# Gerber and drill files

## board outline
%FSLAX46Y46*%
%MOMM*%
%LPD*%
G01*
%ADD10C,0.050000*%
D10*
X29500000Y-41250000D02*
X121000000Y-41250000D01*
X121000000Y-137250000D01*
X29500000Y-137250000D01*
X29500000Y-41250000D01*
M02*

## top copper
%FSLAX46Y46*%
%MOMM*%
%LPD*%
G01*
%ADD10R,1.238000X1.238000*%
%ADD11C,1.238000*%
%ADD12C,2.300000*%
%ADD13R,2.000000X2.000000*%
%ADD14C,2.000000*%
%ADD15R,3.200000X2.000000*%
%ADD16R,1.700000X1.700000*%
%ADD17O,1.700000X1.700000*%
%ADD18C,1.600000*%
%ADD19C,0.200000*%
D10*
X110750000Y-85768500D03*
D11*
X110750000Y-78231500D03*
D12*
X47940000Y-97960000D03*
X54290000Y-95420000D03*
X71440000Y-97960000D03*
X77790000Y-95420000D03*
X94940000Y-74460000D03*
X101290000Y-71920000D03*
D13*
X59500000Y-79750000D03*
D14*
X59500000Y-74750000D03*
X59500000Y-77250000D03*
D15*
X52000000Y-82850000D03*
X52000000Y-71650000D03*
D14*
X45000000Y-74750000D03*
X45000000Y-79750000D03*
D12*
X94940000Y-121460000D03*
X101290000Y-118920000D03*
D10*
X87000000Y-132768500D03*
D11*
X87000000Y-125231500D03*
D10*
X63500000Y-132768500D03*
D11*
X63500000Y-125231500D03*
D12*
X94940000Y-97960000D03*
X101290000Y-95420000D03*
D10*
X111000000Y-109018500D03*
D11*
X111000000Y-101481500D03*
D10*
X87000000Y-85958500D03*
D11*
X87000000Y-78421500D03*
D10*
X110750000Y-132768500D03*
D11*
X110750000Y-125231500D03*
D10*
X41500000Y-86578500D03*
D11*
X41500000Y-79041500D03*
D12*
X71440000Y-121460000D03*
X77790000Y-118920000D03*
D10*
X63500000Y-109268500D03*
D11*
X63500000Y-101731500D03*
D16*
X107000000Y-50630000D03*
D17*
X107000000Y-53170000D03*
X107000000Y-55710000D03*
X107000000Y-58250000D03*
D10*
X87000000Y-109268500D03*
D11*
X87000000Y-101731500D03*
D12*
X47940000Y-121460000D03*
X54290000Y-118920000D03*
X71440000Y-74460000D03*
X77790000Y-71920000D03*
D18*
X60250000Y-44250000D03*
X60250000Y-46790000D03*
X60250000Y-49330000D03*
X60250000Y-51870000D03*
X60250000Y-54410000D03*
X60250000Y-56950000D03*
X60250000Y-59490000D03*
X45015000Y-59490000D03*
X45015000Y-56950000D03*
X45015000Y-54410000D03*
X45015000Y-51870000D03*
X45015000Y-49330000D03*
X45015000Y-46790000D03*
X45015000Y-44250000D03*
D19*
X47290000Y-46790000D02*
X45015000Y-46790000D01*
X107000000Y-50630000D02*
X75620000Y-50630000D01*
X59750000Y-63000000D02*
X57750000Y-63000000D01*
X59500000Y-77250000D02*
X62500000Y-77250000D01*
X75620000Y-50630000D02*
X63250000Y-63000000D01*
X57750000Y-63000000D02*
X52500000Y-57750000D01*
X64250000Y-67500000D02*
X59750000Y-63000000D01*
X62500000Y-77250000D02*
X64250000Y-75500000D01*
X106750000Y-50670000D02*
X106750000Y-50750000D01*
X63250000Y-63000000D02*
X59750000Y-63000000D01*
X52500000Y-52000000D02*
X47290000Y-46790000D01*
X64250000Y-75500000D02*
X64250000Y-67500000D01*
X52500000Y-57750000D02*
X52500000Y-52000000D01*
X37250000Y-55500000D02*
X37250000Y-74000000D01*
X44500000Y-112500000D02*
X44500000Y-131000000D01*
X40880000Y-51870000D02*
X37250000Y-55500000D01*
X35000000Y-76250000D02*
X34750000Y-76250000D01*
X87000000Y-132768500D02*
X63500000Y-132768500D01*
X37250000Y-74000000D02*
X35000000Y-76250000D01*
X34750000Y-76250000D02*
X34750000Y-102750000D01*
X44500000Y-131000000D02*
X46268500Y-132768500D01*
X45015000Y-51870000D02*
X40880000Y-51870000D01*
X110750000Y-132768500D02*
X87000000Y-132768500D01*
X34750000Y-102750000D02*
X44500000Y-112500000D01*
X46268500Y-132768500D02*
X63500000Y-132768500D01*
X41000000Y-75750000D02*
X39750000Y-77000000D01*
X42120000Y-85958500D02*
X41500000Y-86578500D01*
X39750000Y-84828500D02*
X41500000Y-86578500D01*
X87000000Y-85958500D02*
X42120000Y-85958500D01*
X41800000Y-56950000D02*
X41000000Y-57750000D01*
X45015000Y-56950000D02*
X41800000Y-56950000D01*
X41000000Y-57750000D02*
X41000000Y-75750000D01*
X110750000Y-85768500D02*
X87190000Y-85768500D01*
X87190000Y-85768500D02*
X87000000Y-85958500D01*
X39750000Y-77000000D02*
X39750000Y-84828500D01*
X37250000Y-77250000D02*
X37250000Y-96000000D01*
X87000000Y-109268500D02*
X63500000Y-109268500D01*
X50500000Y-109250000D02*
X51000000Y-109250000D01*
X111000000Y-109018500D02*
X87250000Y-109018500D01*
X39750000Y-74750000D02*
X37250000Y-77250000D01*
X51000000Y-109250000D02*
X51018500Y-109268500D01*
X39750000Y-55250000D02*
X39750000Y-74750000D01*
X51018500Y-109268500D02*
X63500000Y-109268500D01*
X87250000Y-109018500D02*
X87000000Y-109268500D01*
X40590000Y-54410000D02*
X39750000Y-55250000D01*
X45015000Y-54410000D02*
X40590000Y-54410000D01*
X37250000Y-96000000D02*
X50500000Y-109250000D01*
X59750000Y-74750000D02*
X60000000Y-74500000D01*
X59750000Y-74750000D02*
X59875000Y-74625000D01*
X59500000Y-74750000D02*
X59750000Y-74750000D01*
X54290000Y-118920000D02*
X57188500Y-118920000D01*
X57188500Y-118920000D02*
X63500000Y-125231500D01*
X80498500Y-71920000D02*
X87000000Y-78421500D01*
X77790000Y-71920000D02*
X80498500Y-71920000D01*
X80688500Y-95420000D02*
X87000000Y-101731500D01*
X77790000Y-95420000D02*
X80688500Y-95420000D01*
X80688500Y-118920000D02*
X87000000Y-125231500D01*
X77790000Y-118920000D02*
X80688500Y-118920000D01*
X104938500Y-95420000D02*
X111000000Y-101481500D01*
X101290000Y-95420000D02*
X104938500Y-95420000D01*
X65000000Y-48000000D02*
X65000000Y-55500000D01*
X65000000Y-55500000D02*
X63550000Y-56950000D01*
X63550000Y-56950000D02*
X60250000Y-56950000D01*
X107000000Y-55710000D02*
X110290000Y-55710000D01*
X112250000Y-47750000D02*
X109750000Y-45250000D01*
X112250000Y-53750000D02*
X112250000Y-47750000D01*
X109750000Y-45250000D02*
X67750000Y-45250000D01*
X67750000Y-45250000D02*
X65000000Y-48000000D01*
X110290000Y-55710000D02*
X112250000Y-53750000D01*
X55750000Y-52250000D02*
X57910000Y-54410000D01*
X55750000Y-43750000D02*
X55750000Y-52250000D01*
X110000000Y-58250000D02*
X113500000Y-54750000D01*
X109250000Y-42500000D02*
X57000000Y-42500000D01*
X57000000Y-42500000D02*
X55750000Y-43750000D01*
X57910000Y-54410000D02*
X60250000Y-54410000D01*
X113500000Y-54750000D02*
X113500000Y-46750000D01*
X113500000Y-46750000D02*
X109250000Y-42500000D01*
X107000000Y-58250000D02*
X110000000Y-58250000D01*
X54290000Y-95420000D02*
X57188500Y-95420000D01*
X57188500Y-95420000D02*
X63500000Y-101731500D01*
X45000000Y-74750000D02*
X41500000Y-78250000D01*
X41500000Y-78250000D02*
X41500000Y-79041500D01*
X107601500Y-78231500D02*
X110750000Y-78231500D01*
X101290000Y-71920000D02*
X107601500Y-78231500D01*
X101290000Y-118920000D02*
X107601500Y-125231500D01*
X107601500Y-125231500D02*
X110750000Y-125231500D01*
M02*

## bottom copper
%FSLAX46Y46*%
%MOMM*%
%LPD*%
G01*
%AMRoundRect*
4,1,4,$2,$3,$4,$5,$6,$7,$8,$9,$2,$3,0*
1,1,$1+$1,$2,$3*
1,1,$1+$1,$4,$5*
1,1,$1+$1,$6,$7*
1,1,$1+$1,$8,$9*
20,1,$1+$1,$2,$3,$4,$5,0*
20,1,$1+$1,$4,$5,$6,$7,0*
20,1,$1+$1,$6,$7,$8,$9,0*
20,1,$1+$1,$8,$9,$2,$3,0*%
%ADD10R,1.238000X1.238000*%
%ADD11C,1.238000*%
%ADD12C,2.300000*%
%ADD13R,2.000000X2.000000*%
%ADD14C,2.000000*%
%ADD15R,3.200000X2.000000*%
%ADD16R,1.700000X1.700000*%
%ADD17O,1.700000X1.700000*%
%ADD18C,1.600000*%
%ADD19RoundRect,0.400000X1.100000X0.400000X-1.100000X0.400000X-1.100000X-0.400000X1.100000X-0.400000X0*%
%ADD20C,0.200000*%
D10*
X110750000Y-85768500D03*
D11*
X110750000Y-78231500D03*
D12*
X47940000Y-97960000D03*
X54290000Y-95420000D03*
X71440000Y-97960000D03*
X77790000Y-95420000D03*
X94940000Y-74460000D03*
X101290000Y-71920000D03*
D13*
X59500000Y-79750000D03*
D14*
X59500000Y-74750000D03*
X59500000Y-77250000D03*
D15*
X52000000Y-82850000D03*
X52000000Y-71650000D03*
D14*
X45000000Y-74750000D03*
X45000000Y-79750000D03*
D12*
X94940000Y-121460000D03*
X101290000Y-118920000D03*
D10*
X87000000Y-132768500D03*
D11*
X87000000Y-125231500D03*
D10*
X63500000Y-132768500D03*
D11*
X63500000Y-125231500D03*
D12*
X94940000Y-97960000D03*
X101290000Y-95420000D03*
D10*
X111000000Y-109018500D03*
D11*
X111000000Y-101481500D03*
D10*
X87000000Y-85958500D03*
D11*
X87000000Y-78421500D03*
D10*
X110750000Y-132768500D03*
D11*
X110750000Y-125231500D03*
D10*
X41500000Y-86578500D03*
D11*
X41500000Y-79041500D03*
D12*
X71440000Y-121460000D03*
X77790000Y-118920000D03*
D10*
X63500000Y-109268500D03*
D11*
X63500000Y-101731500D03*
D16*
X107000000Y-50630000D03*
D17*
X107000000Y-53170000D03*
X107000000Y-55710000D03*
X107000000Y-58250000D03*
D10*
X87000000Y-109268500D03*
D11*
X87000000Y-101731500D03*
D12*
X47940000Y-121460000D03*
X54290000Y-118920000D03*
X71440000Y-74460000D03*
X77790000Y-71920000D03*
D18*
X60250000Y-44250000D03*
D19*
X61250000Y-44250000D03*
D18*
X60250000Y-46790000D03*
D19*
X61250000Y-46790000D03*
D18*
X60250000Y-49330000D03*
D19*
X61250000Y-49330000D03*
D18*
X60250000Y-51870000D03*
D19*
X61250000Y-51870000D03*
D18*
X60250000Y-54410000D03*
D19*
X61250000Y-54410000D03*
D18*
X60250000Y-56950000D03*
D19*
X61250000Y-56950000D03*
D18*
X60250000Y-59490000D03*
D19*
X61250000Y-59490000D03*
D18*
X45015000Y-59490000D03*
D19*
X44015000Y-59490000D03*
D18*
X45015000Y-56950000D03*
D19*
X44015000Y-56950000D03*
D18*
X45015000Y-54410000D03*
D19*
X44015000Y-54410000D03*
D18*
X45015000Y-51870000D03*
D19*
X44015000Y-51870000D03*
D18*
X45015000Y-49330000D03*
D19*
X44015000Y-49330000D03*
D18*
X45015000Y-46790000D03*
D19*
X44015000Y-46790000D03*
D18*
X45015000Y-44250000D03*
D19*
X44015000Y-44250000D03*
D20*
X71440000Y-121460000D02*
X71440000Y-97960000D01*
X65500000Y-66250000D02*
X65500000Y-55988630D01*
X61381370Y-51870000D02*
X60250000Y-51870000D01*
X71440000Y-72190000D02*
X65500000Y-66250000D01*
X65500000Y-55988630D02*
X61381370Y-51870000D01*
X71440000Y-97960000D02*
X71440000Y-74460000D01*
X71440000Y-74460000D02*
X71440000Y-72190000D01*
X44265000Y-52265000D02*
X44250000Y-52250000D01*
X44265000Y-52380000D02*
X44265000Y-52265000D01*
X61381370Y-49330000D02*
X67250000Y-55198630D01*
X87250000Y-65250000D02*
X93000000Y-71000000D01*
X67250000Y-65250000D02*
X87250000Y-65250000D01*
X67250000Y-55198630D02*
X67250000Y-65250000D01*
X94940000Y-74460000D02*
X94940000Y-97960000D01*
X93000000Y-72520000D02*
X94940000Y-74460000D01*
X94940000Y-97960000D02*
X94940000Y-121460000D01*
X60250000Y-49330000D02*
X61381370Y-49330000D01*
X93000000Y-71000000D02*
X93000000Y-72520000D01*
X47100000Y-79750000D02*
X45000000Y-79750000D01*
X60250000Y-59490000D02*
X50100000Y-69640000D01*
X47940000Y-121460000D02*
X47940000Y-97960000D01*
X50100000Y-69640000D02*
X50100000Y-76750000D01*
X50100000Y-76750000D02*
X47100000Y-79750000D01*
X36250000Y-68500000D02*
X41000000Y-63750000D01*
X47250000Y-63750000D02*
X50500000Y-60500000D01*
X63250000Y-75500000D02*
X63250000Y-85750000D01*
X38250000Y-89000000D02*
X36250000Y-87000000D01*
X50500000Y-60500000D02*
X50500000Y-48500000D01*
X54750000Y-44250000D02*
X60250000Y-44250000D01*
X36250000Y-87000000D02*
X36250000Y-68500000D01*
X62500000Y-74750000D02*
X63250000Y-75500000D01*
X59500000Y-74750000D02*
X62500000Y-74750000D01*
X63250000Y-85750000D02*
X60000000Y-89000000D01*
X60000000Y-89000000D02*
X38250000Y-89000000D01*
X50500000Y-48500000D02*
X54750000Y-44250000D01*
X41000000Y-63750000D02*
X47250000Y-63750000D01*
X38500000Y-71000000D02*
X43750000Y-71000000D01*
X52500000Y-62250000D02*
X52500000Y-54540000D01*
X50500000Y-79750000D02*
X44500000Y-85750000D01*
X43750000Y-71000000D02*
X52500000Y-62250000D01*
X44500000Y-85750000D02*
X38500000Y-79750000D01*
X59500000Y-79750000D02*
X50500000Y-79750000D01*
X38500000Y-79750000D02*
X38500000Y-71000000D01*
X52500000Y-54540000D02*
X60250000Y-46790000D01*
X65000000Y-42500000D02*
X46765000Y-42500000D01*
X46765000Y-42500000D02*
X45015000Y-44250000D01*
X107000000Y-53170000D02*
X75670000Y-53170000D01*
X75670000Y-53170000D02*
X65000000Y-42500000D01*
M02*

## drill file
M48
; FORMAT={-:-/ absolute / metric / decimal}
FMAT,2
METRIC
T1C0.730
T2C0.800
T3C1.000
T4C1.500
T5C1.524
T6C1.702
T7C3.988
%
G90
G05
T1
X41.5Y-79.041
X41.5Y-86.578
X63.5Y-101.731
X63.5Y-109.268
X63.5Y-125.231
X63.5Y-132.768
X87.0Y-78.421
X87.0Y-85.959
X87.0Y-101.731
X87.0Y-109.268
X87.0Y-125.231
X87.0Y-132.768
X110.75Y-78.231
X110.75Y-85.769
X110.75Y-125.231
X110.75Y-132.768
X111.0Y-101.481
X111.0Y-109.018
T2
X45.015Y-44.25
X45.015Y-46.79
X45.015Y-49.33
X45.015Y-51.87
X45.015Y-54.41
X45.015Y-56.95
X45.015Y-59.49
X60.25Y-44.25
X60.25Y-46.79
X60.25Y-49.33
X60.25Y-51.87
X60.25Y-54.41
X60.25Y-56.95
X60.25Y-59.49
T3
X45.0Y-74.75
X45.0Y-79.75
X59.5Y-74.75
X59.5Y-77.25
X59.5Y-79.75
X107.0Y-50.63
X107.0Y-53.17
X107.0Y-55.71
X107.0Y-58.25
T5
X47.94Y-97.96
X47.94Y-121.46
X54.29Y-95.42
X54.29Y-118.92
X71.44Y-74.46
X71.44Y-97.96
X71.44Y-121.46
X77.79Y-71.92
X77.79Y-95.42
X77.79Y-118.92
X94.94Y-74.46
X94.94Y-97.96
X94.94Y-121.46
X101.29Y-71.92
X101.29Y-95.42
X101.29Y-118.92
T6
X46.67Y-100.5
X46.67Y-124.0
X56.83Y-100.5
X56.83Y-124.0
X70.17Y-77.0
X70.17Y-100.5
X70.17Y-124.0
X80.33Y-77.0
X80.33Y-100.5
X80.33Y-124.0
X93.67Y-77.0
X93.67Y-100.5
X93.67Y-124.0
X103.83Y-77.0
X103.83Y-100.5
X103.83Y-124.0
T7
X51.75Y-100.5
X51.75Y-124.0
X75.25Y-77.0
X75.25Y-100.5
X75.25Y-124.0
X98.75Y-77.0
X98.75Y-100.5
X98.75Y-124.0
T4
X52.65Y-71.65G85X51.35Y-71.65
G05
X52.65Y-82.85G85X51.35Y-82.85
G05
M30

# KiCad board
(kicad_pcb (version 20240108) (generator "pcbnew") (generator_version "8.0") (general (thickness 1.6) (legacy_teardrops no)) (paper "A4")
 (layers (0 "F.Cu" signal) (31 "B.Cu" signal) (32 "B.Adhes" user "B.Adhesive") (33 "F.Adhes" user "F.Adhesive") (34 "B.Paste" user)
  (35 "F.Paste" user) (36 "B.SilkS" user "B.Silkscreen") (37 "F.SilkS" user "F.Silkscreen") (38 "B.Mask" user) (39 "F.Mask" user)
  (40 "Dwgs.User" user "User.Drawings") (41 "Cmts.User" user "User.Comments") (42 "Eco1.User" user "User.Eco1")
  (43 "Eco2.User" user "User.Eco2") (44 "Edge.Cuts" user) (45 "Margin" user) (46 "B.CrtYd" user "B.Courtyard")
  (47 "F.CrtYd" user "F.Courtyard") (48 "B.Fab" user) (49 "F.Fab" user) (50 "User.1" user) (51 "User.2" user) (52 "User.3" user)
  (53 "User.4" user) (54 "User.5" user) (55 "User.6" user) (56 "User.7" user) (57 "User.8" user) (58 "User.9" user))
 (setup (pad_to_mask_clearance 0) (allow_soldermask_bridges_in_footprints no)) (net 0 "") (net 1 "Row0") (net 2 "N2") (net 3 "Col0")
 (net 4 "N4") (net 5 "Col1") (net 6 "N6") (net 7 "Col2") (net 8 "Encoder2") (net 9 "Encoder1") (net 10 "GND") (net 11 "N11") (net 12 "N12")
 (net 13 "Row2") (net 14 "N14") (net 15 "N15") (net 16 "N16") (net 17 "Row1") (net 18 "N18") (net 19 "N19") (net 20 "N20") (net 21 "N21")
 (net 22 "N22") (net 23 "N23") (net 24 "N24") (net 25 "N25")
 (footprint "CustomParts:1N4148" (layer "F.Cu") (at 110.75 82 90)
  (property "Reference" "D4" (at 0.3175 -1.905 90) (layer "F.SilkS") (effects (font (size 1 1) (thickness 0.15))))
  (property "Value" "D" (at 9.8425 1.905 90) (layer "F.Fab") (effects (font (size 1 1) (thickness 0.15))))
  (pad "1" thru_hole rect (at -3.7685 0 90) (size 1.238 1.238) (drill 0.73) (layers "*.Cu" "*.Mask") (remove_unused_layers no)
   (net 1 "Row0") (solder_mask_margin 0.102))
  (pad "2" thru_hole circle (at 3.7685 0 90) (size 1.238 1.238) (drill 0.73) (layers "*.Cu" "*.Mask") (remove_unused_layers no) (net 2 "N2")
   (solder_mask_margin 0.102)))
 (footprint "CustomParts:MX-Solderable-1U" (layer "F.Cu") (at 51.75 100.5)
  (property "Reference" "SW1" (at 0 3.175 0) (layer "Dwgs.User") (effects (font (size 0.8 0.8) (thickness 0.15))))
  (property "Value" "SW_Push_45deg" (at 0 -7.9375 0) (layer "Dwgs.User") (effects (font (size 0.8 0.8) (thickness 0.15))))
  (pad "" np_thru_hole circle (at -5.08 0 48.099) (size 1.7018 1.7018) (drill 1.7018) (layers "F&B.Cu" "*.Mask"))
  (pad "" np_thru_hole circle (at 0 0) (size 3.9878 3.9878) (drill 3.9878) (layers "*.Cu" "*.Mask"))
  (pad "" np_thru_hole circle (at 5.08 0 48.099) (size 1.7018 1.7018) (drill 1.7018) (layers "F&B.Cu" "*.Mask"))
  (pad "1" thru_hole circle (at -3.81 -2.54) (size 2.3 2.3) (drill 1.524) (layers "*.Cu" "B.Mask") (remove_unused_layers no) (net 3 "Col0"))
  (pad "2" thru_hole circle (at 2.54 -5.08) (size 2.3 2.3) (drill 1.524) (layers "*.Cu" "B.Mask") (remove_unused_layers no) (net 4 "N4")))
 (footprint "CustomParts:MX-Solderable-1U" (layer "F.Cu") (at 75.25 100.5)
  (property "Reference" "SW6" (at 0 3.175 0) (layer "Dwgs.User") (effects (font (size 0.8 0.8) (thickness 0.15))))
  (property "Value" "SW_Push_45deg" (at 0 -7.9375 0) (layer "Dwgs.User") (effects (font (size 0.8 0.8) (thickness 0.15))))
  (pad "" np_thru_hole circle (at -5.08 0 48.099) (size 1.7018 1.7018) (drill 1.7018) (layers "F&B.Cu" "*.Mask"))
  (pad "" np_thru_hole circle (at 0 0) (size 3.9878 3.9878) (drill 3.9878) (layers "*.Cu" "*.Mask"))
  (pad "" np_thru_hole circle (at 5.08 0 48.099) (size 1.7018 1.7018) (drill 1.7018) (layers "F&B.Cu" "*.Mask"))
  (pad "1" thru_hole circle (at -3.81 -2.54) (size 2.3 2.3) (drill 1.524) (layers "*.Cu" "B.Mask") (remove_unused_layers no) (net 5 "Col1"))
  (pad "2" thru_hole circle (at 2.54 -5.08) (size 2.3 2.3) (drill 1.524) (layers "*.Cu" "B.Mask") (remove_unused_layers no) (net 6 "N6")))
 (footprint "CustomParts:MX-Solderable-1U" (layer "F.Cu") (at 98.75 77)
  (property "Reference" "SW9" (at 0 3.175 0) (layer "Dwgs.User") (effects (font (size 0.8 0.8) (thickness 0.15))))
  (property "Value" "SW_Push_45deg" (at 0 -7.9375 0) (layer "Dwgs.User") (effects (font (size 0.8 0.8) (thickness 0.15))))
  (pad "" np_thru_hole circle (at -5.08 0 48.099) (size 1.7018 1.7018) (drill 1.7018) (layers "F&B.Cu" "*.Mask"))
  (pad "" np_thru_hole circle (at 0 0) (size 3.9878 3.9878) (drill 3.9878) (layers "*.Cu" "*.Mask"))
  (pad "" np_thru_hole circle (at 5.08 0 48.099) (size 1.7018 1.7018) (drill 1.7018) (layers "F&B.Cu" "*.Mask"))
  (pad "1" thru_hole circle (at -3.81 -2.54) (size 2.3 2.3) (drill 1.524) (layers "*.Cu" "B.Mask") (remove_unused_layers no) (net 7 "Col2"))
  (pad "2" thru_hole circle (at 2.54 -5.08) (size 2.3 2.3) (drill 1.524) (layers "*.Cu" "B.Mask") (remove_unused_layers no) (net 2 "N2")))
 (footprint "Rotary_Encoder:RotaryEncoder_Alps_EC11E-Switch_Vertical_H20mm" (layer "F.Cu") (at 59.5 79.75 180)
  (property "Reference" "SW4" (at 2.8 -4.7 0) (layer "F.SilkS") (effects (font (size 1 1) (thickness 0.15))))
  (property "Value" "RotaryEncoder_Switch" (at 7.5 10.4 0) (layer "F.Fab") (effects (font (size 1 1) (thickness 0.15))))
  (pad "A" thru_hole rect (at 0 0 180) (size 2 2) (drill 1) (layers "*.Cu" "*.Mask") (remove_unused_layers no) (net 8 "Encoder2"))
  (pad "B" thru_hole circle (at 0 5 180) (size 2 2) (drill 1) (layers "*.Cu" "*.Mask") (remove_unused_layers no) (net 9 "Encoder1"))
  (pad "C" thru_hole circle (at 0 2.5 180) (size 2 2) (drill 1) (layers "*.Cu" "*.Mask") (remove_unused_layers no) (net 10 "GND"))
  (pad "MP" thru_hole rect (at 7.5 -3.1 180) (size 3.2 2) (drill oval 2.8 1.5) (layers "*.Cu" "*.Mask") (remove_unused_layers no))
  (pad "MP" thru_hole rect (at 7.5 8.1 180) (size 3.2 2) (drill oval 2.8 1.5) (layers "*.Cu" "*.Mask") (remove_unused_layers no))
  (pad "S1" thru_hole circle (at 14.5 5 180) (size 2 2) (drill 1) (layers "*.Cu" "*.Mask") (remove_unused_layers no) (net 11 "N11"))
  (pad "S2" thru_hole circle (at 14.5 0 180) (size 2 2) (drill 1) (layers "*.Cu" "*.Mask") (remove_unused_layers no) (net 3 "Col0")))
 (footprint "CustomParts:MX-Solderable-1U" (layer "F.Cu") (at 98.75 124)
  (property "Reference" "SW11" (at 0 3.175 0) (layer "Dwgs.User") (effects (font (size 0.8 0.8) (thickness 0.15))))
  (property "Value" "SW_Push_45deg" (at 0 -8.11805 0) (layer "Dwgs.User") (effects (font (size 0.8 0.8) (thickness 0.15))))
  (pad "" np_thru_hole circle (at -5.08 0 48.099) (size 1.7018 1.7018) (drill 1.7018) (layers "F&B.Cu" "*.Mask"))
  (pad "" np_thru_hole circle (at 0 0) (size 3.9878 3.9878) (drill 3.9878) (layers "*.Cu" "*.Mask"))
  (pad "" np_thru_hole circle (at 5.08 0 48.099) (size 1.7018 1.7018) (drill 1.7018) (layers "F&B.Cu" "*.Mask"))
  (pad "1" thru_hole circle (at -3.81 -2.54) (size 2.3 2.3) (drill 1.524) (layers "*.Cu" "B.Mask") (remove_unused_layers no) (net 7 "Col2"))
  (pad "2" thru_hole circle (at 2.54 -5.08) (size 2.3 2.3) (drill 1.524) (layers "*.Cu" "B.Mask") (remove_unused_layers no) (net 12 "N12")))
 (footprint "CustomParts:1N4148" (layer "F.Cu") (at 87 129 90)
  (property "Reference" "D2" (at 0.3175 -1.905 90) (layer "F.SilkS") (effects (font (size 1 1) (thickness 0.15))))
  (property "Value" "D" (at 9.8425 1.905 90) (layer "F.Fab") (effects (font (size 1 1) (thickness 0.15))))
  (pad "1" thru_hole rect (at -3.7685 0 90) (size 1.238 1.238) (drill 0.73) (layers "*.Cu" "*.Mask") (remove_unused_layers no)
   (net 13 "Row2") (solder_mask_margin 0.102))
  (pad "2" thru_hole circle (at 3.7685 0 90) (size 1.238 1.238) (drill 0.73) (layers "*.Cu" "*.Mask") (remove_unused_layers no)
   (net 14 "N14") (solder_mask_margin 0.102)))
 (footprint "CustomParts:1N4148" (layer "F.Cu") (at 63.5 129 90)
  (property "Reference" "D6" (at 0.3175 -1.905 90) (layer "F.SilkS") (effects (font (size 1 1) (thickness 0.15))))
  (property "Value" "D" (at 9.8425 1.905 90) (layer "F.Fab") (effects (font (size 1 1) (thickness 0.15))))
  (pad "1" thru_hole rect (at -3.7685 0 90) (size 1.238 1.238) (drill 0.73) (layers "*.Cu" "*.Mask") (remove_unused_layers no)
   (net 13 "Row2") (solder_mask_margin 0.102))
  (pad "2" thru_hole circle (at 3.7685 0 90) (size 1.238 1.238) (drill 0.73) (layers "*.Cu" "*.Mask") (remove_unused_layers no)
   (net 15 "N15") (solder_mask_margin 0.102)))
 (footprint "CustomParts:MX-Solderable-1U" (layer "F.Cu") (at 98.75 100.5)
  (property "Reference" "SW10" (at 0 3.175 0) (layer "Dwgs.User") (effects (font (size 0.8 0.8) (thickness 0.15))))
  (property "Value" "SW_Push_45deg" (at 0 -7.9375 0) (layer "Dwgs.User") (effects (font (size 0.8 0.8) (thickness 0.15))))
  (pad "" np_thru_hole circle (at -5.08 0 48.099) (size 1.7018 1.7018) (drill 1.7018) (layers "F&B.Cu" "*.Mask"))
  (pad "" np_thru_hole circle (at 0 0) (size 3.9878 3.9878) (drill 3.9878) (layers "*.Cu" "*.Mask"))
  (pad "" np_thru_hole circle (at 5.08 0 48.099) (size 1.7018 1.7018) (drill 1.7018) (layers "F&B.Cu" "*.Mask"))
  (pad "1" thru_hole circle (at -3.81 -2.54) (size 2.3 2.3) (drill 1.524) (layers "*.Cu" "B.Mask") (remove_unused_layers no) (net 7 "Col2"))
  (pad "2" thru_hole circle (at 2.54 -5.08) (size 2.3 2.3) (drill 1.524) (layers "*.Cu" "B.Mask") (remove_unused_layers no) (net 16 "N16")))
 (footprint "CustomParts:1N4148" (layer "F.Cu") (at 111 105.25 90)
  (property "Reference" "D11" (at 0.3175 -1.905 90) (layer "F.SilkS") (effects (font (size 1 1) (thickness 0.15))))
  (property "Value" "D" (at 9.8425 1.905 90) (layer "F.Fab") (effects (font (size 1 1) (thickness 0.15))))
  (pad "1" thru_hole rect (at -3.7685 0 90) (size 1.238 1.238) (drill 0.73) (layers "*.Cu" "*.Mask") (remove_unused_layers no)
   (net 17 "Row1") (solder_mask_margin 0.102))
  (pad "2" thru_hole circle (at 3.7685 0 90) (size 1.238 1.238) (drill 0.73) (layers "*.Cu" "*.Mask") (remove_unused_layers no)
   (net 16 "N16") (solder_mask_margin 0.102)))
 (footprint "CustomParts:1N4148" (layer "F.Cu") (at 87 82.19 90)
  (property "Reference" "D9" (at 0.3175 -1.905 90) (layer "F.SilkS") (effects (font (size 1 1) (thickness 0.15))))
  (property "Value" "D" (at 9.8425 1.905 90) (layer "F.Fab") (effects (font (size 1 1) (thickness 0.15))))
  (pad "1" thru_hole rect (at -3.7685 0 90) (size 1.238 1.238) (drill 0.73) (layers "*.Cu" "*.Mask") (remove_unused_layers no)
   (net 1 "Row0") (solder_mask_margin 0.102))
  (pad "2" thru_hole circle (at 3.7685 0 90) (size 1.238 1.238) (drill 0.73) (layers "*.Cu" "*.Mask") (remove_unused_layers no)
   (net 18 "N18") (solder_mask_margin 0.102)))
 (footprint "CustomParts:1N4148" (layer "F.Cu") (at 110.75 129 90)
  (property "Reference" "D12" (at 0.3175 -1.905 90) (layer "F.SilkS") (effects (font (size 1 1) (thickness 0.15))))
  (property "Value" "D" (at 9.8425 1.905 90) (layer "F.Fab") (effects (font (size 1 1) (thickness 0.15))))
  (pad "1" thru_hole rect (at -3.7685 0 90) (size 1.238 1.238) (drill 0.73) (layers "*.Cu" "*.Mask") (remove_unused_layers no)
   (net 13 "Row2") (solder_mask_margin 0.102))
  (pad "2" thru_hole circle (at 3.7685 0 90) (size 1.238 1.238) (drill 0.73) (layers "*.Cu" "*.Mask") (remove_unused_layers no)
   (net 12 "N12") (solder_mask_margin 0.102)))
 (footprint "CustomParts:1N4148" (layer "F.Cu") (at 41.5 82.81 90)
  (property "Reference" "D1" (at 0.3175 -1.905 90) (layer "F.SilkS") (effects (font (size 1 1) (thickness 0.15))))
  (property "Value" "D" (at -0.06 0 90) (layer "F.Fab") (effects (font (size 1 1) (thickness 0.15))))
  (pad "1" thru_hole rect (at -3.7685 0 90) (size 1.238 1.238) (drill 0.73) (layers "*.Cu" "*.Mask") (remove_unused_layers no)
   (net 1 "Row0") (solder_mask_margin 0.102))
  (pad "2" thru_hole circle (at 3.7685 0 90) (size 1.238 1.238) (drill 0.73) (layers "*.Cu" "*.Mask") (remove_unused_layers no)
   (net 11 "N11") (solder_mask_margin 0.102)))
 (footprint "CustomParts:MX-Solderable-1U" (layer "F.Cu") (at 75.25 124)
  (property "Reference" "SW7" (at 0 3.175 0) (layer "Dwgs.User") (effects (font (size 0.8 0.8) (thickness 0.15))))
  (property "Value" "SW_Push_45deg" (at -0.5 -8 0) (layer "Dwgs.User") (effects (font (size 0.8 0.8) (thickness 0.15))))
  (pad "" np_thru_hole circle (at -5.08 0 48.099) (size 1.7018 1.7018) (drill 1.7018) (layers "F&B.Cu" "*.Mask"))
  (pad "" np_thru_hole circle (at 0 0) (size 3.9878 3.9878) (drill 3.9878) (layers "*.Cu" "*.Mask"))
  (pad "" np_thru_hole circle (at 5.08 0 48.099) (size 1.7018 1.7018) (drill 1.7018) (layers "F&B.Cu" "*.Mask"))
  (pad "1" thru_hole circle (at -3.81 -2.54) (size 2.3 2.3) (drill 1.524) (layers "*.Cu" "B.Mask") (remove_unused_layers no) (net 5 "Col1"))
  (pad "2" thru_hole circle (at 2.54 -5.08) (size 2.3 2.3) (drill 1.524) (layers "*.Cu" "B.Mask") (remove_unused_layers no) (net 14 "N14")))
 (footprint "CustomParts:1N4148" (layer "F.Cu") (at 63.5 105.5 90)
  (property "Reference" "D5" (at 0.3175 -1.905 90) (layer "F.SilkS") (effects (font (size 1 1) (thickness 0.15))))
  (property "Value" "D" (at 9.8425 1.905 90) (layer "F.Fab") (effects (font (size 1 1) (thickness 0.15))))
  (pad "1" thru_hole rect (at -3.7685 0 90) (size 1.238 1.238) (drill 0.73) (layers "*.Cu" "*.Mask") (remove_unused_layers no)
   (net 17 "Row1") (solder_mask_margin 0.102))
  (pad "2" thru_hole circle (at 3.7685 0 90) (size 1.238 1.238) (drill 0.73) (layers "*.Cu" "*.Mask") (remove_unused_layers no) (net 4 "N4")
   (solder_mask_margin 0.102)))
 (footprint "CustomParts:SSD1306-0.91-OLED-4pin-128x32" (layer "F.Cu") (at 70.5 48.44)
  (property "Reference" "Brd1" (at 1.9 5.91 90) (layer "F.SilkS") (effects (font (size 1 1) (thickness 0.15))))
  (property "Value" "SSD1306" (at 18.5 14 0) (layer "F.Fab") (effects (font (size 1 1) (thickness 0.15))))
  (pad "1" thru_hole rect (at 36.5 2.19) (size 1.7 1.7) (drill 1) (layers "*.Cu" "*.Mask") (remove_unused_layers no) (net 10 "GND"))
  (pad "2" thru_hole oval (at 36.5 4.73) (size 1.7 1.7) (drill 1) (layers "*.Cu" "*.Mask") (remove_unused_layers no) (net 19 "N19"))
  (pad "3" thru_hole oval (at 36.5 7.27) (size 1.7 1.7) (drill 1) (layers "*.Cu" "*.Mask") (remove_unused_layers no) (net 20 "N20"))
  (pad "4" thru_hole oval (at 36.5 9.81) (size 1.7 1.7) (drill 1) (layers "*.Cu" "*.Mask") (remove_unused_layers no) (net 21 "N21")))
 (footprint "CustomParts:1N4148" (layer "F.Cu") (at 87 105.5 90)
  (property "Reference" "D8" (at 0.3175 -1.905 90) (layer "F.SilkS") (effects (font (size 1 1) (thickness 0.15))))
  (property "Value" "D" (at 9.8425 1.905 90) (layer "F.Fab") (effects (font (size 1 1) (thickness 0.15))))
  (pad "1" thru_hole rect (at -3.7685 0 90) (size 1.238 1.238) (drill 0.73) (layers "*.Cu" "*.Mask") (remove_unused_layers no)
   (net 17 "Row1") (solder_mask_margin 0.102))
  (pad "2" thru_hole circle (at 3.7685 0 90) (size 1.238 1.238) (drill 0.73) (layers "*.Cu" "*.Mask") (remove_unused_layers no) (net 6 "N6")
   (solder_mask_margin 0.102)))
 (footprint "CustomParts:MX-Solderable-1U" (layer "F.Cu") (at 51.75 124)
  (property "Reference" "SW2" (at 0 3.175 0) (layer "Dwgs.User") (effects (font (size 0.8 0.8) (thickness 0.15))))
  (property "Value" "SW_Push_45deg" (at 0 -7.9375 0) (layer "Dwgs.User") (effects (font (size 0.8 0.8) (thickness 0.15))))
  (pad "" np_thru_hole circle (at -5.08 0 48.099) (size 1.7018 1.7018) (drill 1.7018) (layers "F&B.Cu" "*.Mask"))
  (pad "" np_thru_hole circle (at 0 0) (size 3.9878 3.9878) (drill 3.9878) (layers "*.Cu" "*.Mask"))
  (pad "" np_thru_hole circle (at 5.08 0 48.099) (size 1.7018 1.7018) (drill 1.7018) (layers "F&B.Cu" "*.Mask"))
  (pad "1" thru_hole circle (at -3.81 -2.54) (size 2.3 2.3) (drill 1.524) (layers "*.Cu" "B.Mask") (remove_unused_layers no) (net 3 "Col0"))
  (pad "2" thru_hole circle (at 2.54 -5.08) (size 2.3 2.3) (drill 1.524) (layers "*.Cu" "B.Mask") (remove_unused_layers no) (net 15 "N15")))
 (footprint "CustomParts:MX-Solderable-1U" (layer "F.Cu") (at 75.25 77)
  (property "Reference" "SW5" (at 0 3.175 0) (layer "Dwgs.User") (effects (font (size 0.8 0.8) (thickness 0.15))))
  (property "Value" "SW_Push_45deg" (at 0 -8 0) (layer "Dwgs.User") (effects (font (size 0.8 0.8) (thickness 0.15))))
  (pad "" np_thru_hole circle (at -5.08 0 48.099) (size 1.7018 1.7018) (drill 1.7018) (layers "F&B.Cu" "*.Mask"))
  (pad "" np_thru_hole circle (at 0 0) (size 3.9878 3.9878) (drill 3.9878) (layers "*.Cu" "*.Mask"))
  (pad "" np_thru_hole circle (at 5.08 0 48.099) (size 1.7018 1.7018) (drill 1.7018) (layers "F&B.Cu" "*.Mask"))
  (pad "1" thru_hole circle (at -3.81 -2.54) (size 2.3 2.3) (drill 1.524) (layers "*.Cu" "B.Mask") (remove_unused_layers no) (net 5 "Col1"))
  (pad "2" thru_hole circle (at 2.54 -5.08) (size 2.3 2.3) (drill 1.524) (layers "*.Cu" "B.Mask") (remove_unused_layers no) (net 18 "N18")))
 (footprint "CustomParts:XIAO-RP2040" (layer "B.Cu") (at 61.5225 62.421 180)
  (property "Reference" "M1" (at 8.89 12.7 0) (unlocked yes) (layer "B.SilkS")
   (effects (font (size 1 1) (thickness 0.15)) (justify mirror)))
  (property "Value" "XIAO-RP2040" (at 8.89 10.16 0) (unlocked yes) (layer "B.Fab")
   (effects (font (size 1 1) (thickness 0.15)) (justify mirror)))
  (pad "1" thru_hole circle (at 1.2725 18.171 180) (size 1.6 1.6) (drill 0.8) (layers "*.Cu" "*.Mask") (remove_unused_layers no)
   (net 9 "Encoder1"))
  (pad "1" smd roundrect (at 1.2725 18.171 180) (size 3 1.6) (drill (offset -1 0)) (layers "B.Cu" "B.Paste" "B.Mask")
   (roundrect_rratio 0.25) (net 9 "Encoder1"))
  (pad "2" thru_hole circle (at 1.2725 15.631 180) (size 1.6 1.6) (drill 0.8) (layers "*.Cu" "*.Mask") (remove_unused_layers no)
   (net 8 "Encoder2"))
  (pad "2" smd roundrect (at 1.2725 15.631 180) (size 3 1.6) (drill (offset -1 0)) (layers "B.Cu" "B.Paste" "B.Mask")
   (roundrect_rratio 0.25) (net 8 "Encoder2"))
  (pad "3" thru_hole circle (at 1.2725 13.091 180) (size 1.6 1.6) (drill 0.8) (layers "*.Cu" "*.Mask") (remove_unused_layers no)
   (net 7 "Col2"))
  (pad "3" smd roundrect (at 1.2725 13.091 180) (size 3 1.6) (drill (offset -1 0)) (layers "B.Cu" "B.Paste" "B.Mask")
   (roundrect_rratio 0.25) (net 7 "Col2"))
  (pad "4" thru_hole circle (at 1.2725 10.551 180) (size 1.6 1.6) (drill 0.8) (layers "*.Cu" "*.Mask") (remove_unused_layers no)
   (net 5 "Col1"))
  (pad "4" smd roundrect (at 1.2725 10.551 180) (size 3 1.6) (drill (offset -1 0)) (layers "B.Cu" "B.Paste" "B.Mask")
   (roundrect_rratio 0.25) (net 5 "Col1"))
  (pad "5" thru_hole circle (at 1.2725 8.011 180) (size 1.6 1.6) (drill 0.8) (layers "*.Cu" "*.Mask") (remove_unused_layers no)
   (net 21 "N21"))
  (pad "5" smd roundrect (at 1.2725 8.011 180) (size 3 1.6) (drill (offset -1 0)) (layers "B.Cu" "B.Paste" "B.Mask") (roundrect_rratio 0.25)
   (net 21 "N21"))
  (pad "6" thru_hole circle (at 1.2725 5.471 180) (size 1.6 1.6) (drill 0.8) (layers "*.Cu" "*.Mask") (remove_unused_layers no)
   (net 20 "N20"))
  (pad "6" smd roundrect (at 1.2725 5.471 180) (size 3 1.6) (drill (offset -1 0)) (layers "B.Cu" "B.Paste" "B.Mask") (roundrect_rratio 0.25)
   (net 20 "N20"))
  (pad "7" thru_hole circle (at 1.2725 2.931 180) (size 1.6 1.6) (drill 0.8) (layers "*.Cu" "*.Mask") (remove_unused_layers no)
   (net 3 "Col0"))
  (pad "7" smd roundrect (at 1.2725 2.931 180) (size 3 1.6) (drill (offset -1 0)) (layers "B.Cu" "B.Paste" "B.Mask") (roundrect_rratio 0.25)
   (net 3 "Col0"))
  (pad "8" thru_hole circle (at 16.5075 2.931 180) (size 1.6 1.6) (drill 0.8) (layers "*.Cu" "*.Mask") (remove_unused_layers no)
   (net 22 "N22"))
  (pad "8" smd roundrect (at 16.5075 2.931 180) (size 3 1.6) (drill (offset 1 0)) (layers "B.Cu" "B.Paste" "B.Mask") (roundrect_rratio 0.25)
   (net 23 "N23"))
  (pad "9" thru_hole circle (at 16.5075 5.471 180) (size 1.6 1.6) (drill 0.8) (layers "*.Cu" "*.Mask") (remove_unused_layers no)
   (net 1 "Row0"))
  (pad "9" smd roundrect (at 16.5075 5.471 180) (size 3 1.6) (drill (offset 1 0)) (layers "B.Cu" "B.Paste" "B.Mask") (roundrect_rratio 0.25)
   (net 1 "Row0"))
  (pad "10" thru_hole circle (at 16.5075 8.011 180) (size 1.6 1.6) (drill 0.8) (layers "*.Cu" "*.Mask") (remove_unused_layers no)
   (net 17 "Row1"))
  (pad "10" smd roundrect (at 16.5075 8.011 180) (size 3 1.6) (drill (offset 1 0)) (layers "B.Cu" "B.Paste" "B.Mask")
   (roundrect_rratio 0.25) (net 17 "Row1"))
  (pad "11" thru_hole circle (at 16.5075 10.551 180) (size 1.6 1.6) (drill 0.8) (layers "*.Cu" "*.Mask") (remove_unused_layers no)
   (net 13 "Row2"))
  (pad "11" smd roundrect (at 16.5075 10.551 180) (size 3 1.6) (drill (offset 1 0)) (layers "B.Cu" "B.Paste" "B.Mask")
   (roundrect_rratio 0.25) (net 13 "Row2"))
  (pad "12" thru_hole circle (at 16.5075 13.091 180) (size 1.6 1.6) (drill 0.8) (layers "*.Cu" "*.Mask") (remove_unused_layers no)
   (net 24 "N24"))
  (pad "12" smd roundrect (at 16.5075 13.091 180) (size 3 1.6) (drill (offset 1 0)) (layers "B.Cu" "B.Paste" "B.Mask")
   (roundrect_rratio 0.25) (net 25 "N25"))
  (pad "13" thru_hole circle (at 16.5075 15.631 180) (size 1.6 1.6) (drill 0.8) (layers "*.Cu" "*.Mask") (remove_unused_layers no)
   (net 10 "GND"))
  (pad "13" smd roundrect (at 16.5075 15.631 180) (size 3 1.6) (drill (offset 1 0)) (layers "B.Cu" "B.Paste" "B.Mask")
   (roundrect_rratio 0.25) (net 10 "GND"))
  (pad "14" thru_hole circle (at 16.5075 18.171 180) (size 1.6 1.6) (drill 0.8) (layers "*.Cu" "*.Mask") (remove_unused_layers no)
   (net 19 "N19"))
  (pad "14" smd roundrect (at 16.5075 18.171 180) (size 3 1.6) (drill (offset 1 0)) (layers "B.Cu" "B.Paste" "B.Mask")
   (roundrect_rratio 0.25) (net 19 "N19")))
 (gr_rect (start 29.5 41.25) (end 121 137.25) (stroke (width 0.05) (type default)) (fill none) (layer "Edge.Cuts"))
 (segment (start 71.44 121.46) (end 71.44 97.96) (width 0.2) (layer "B.Cu") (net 5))
 (segment (start 65.5 66.25) (end 65.5 55.98863) (width 0.2) (layer "B.Cu") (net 5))
 (segment (start 61.38137 51.87) (end 60.25 51.87) (width 0.2) (layer "B.Cu") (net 5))
 (segment (start 71.44 72.19) (end 65.5 66.25) (width 0.2) (layer "B.Cu") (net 5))
 (segment (start 65.5 55.98863) (end 61.38137 51.87) (width 0.2) (layer "B.Cu") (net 5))
 (segment (start 71.44 97.96) (end 71.44 74.46) (width 0.2) (layer "B.Cu") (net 5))
 (segment (start 71.44 74.46) (end 71.44 72.19) (width 0.2) (layer "B.Cu") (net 5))
 (segment (start 47.29 46.79) (end 45.015 46.79) (width 0.2) (layer "F.Cu") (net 10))
 (segment (start 107 50.63) (end 75.62 50.63) (width 0.2) (layer "F.Cu") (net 10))
 (segment (start 59.75 63) (end 57.75 63) (width 0.2) (layer "F.Cu") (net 10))
 (segment (start 59.5 77.25) (end 62.5 77.25) (width 0.2) (layer "F.Cu") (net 10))
 (segment (start 75.62 50.63) (end 63.25 63) (width 0.2) (layer "F.Cu") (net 10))
 (segment (start 57.75 63) (end 52.5 57.75) (width 0.2) (layer "F.Cu") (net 10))
 (segment (start 64.25 67.5) (end 59.75 63) (width 0.2) (layer "F.Cu") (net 10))
 (segment (start 62.5 77.25) (end 64.25 75.5) (width 0.2) (layer "F.Cu") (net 10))
 (segment (start 106.75 50.67) (end 106.75 50.75) (width 0.2) (layer "F.Cu") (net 10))
 (segment (start 63.25 63) (end 59.75 63) (width 0.2) (layer "F.Cu") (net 10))
 (segment (start 52.5 52) (end 47.29 46.79) (width 0.2) (layer "F.Cu") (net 10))
 (segment (start 64.25 75.5) (end 64.25 67.5) (width 0.2) (layer "F.Cu") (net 10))
 (segment (start 52.5 57.75) (end 52.5 52) (width 0.2) (layer "F.Cu") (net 10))
 (segment (start 37.25 55.5) (end 37.25 74) (width 0.2) (layer "F.Cu") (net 13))
 (segment (start 44.5 112.5) (end 44.5 131) (width 0.2) (layer "F.Cu") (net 13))
 (segment (start 40.88 51.87) (end 37.25 55.5) (width 0.2) (layer "F.Cu") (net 13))
 (segment (start 35 76.25) (end 34.75 76.25) (width 0.2) (layer "F.Cu") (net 13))
 (segment (start 87 132.7685) (end 63.5 132.7685) (width 0.2) (layer "F.Cu") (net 13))
 (segment (start 37.25 74) (end 35 76.25) (width 0.2) (layer "F.Cu") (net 13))
 (segment (start 34.75 76.25) (end 34.75 102.75) (width 0.2) (layer "F.Cu") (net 13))
 (segment (start 44.5 131) (end 46.2685 132.7685) (width 0.2) (layer "F.Cu") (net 13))
 (segment (start 45.015 51.87) (end 40.88 51.87) (width 0.2) (layer "F.Cu") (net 13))
 (segment (start 110.75 132.7685) (end 87 132.7685) (width 0.2) (layer "F.Cu") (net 13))
 (segment (start 34.75 102.75) (end 44.5 112.5) (width 0.2) (layer "F.Cu") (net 13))
 (segment (start 46.2685 132.7685) (end 63.5 132.7685) (width 0.2) (layer "F.Cu") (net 13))
 (segment (start 44.265 52.265) (end 44.25 52.25) (width 0.2) (layer "B.Cu") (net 13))
 (segment (start 44.265 52.38) (end 44.265 52.265) (width 0.2) (layer "B.Cu") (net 13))
 (segment (start 61.38137 49.33) (end 67.25 55.19863) (width 0.2) (layer "B.Cu") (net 7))
 (segment (start 87.25 65.25) (end 93 71) (width 0.2) (layer "B.Cu") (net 7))
 (segment (start 67.25 65.25) (end 87.25 65.25) (width 0.2) (layer "B.Cu") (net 7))
 (segment (start 67.25 55.19863) (end 67.25 65.25) (width 0.2) (layer "B.Cu") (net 7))
 (segment (start 94.94 74.46) (end 94.94 97.96) (width 0.2) (layer "B.Cu") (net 7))
 (segment (start 93 72.52) (end 94.94 74.46) (width 0.2) (layer "B.Cu") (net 7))
 (segment (start 94.94 97.96) (end 94.94 121.46) (width 0.2) (layer "B.Cu") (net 7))
 (segment (start 60.25 49.33) (end 61.38137 49.33) (width 0.2) (layer "B.Cu") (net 7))
 (segment (start 93 71) (end 93 72.52) (width 0.2) (layer "B.Cu") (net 7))
 (segment (start 47.1 79.75) (end 45 79.75) (width 0.2) (layer "B.Cu") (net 3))
 (segment (start 60.25 59.49) (end 50.1 69.64) (width 0.2) (layer "B.Cu") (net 3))
 (segment (start 47.94 121.46) (end 47.94 97.96) (width 0.2) (layer "B.Cu") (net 3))
 (segment (start 50.1 69.64) (end 50.1 76.75) (width 0.2) (layer "B.Cu") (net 3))
 (segment (start 50.1 76.75) (end 47.1 79.75) (width 0.2) (layer "B.Cu") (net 3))
 (segment (start 41 75.75) (end 39.75 77) (width 0.2) (layer "F.Cu") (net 1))
 (segment (start 42.12 85.9585) (end 41.5 86.5785) (width 0.2) (layer "F.Cu") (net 1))
 (segment (start 39.75 84.8285) (end 41.5 86.5785) (width 0.2) (layer "F.Cu") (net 1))
 (segment (start 87 85.9585) (end 42.12 85.9585) (width 0.2) (layer "F.Cu") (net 1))
 (segment (start 41.8 56.95) (end 41 57.75) (width 0.2) (layer "F.Cu") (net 1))
 (segment (start 45.015 56.95) (end 41.8 56.95) (width 0.2) (layer "F.Cu") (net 1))
 (segment (start 41 57.75) (end 41 75.75) (width 0.2) (layer "F.Cu") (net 1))
 (segment (start 110.75 85.7685) (end 87.19 85.7685) (width 0.2) (layer "F.Cu") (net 1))
 (segment (start 87.19 85.7685) (end 87 85.9585) (width 0.2) (layer "F.Cu") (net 1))
 (segment (start 39.75 77) (end 39.75 84.8285) (width 0.2) (layer "F.Cu") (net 1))
 (segment (start 37.25 77.25) (end 37.25 96) (width 0.2) (layer "F.Cu") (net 17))
 (segment (start 87 109.2685) (end 63.5 109.2685) (width 0.2) (layer "F.Cu") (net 17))
 (segment (start 50.5 109.25) (end 51 109.25) (width 0.2) (layer "F.Cu") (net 17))
 (segment (start 111 109.0185) (end 87.25 109.0185) (width 0.2) (layer "F.Cu") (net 17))
 (segment (start 39.75 74.75) (end 37.25 77.25) (width 0.2) (layer "F.Cu") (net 17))
 (segment (start 51 109.25) (end 51.0185 109.2685) (width 0.2) (layer "F.Cu") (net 17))
 (segment (start 39.75 55.25) (end 39.75 74.75) (width 0.2) (layer "F.Cu") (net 17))
 (segment (start 51.0185 109.2685) (end 63.5 109.2685) (width 0.2) (layer "F.Cu") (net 17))
 (segment (start 87.25 109.0185) (end 87 109.2685) (width 0.2) (layer "F.Cu") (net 17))
 (segment (start 40.59 54.41) (end 39.75 55.25) (width 0.2) (layer "F.Cu") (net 17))
 (segment (start 45.015 54.41) (end 40.59 54.41) (width 0.2) (layer "F.Cu") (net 17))
 (segment (start 37.25 96) (end 50.5 109.25) (width 0.2) (layer "F.Cu") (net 17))
 (segment (start 59.75 74.75) (end 60 74.5) (width 0.2) (layer "F.Cu") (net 9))
 (segment (start 59.75 74.75) (end 59.875 74.625) (width 0.2) (layer "F.Cu") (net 9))
 (segment (start 59.5 74.75) (end 59.75 74.75) (width 0.2) (layer "F.Cu") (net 9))
 (segment (start 36.25 68.5) (end 41 63.75) (width 0.2) (layer "B.Cu") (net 9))
 (segment (start 47.25 63.75) (end 50.5 60.5) (width 0.2) (layer "B.Cu") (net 9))
 (segment (start 63.25 75.5) (end 63.25 85.75) (width 0.2) (layer "B.Cu") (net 9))
 (segment (start 38.25 89) (end 36.25 87) (width 0.2) (layer "B.Cu") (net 9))
 (segment (start 50.5 60.5) (end 50.5 48.5) (width 0.2) (layer "B.Cu") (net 9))
 (segment (start 54.75 44.25) (end 60.25 44.25) (width 0.2) (layer "B.Cu") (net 9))
 (segment (start 36.25 87) (end 36.25 68.5) (width 0.2) (layer "B.Cu") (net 9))
 (segment (start 62.5 74.75) (end 63.25 75.5) (width 0.2) (layer "B.Cu") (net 9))
 (segment (start 59.5 74.75) (end 62.5 74.75) (width 0.2) (layer "B.Cu") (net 9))
 (segment (start 63.25 85.75) (end 60 89) (width 0.2) (layer "B.Cu") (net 9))
 (segment (start 60 89) (end 38.25 89) (width 0.2) (layer "B.Cu") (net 9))
 (segment (start 50.5 48.5) (end 54.75 44.25) (width 0.2) (layer "B.Cu") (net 9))
 (segment (start 41 63.75) (end 47.25 63.75) (width 0.2) (layer "B.Cu") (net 9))
 (segment (start 38.5 71) (end 43.75 71) (width 0.2) (layer "B.Cu") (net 8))
 (segment (start 52.5 62.25) (end 52.5 54.54) (width 0.2) (layer "B.Cu") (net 8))
 (segment (start 50.5 79.75) (end 44.5 85.75) (width 0.2) (layer "B.Cu") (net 8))
 (segment (start 43.75 71) (end 52.5 62.25) (width 0.2) (layer "B.Cu") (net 8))
 (segment (start 44.5 85.75) (end 38.5 79.75) (width 0.2) (layer "B.Cu") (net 8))
 (segment (start 59.5 79.75) (end 50.5 79.75) (width 0.2) (layer "B.Cu") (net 8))
 (segment (start 38.5 79.75) (end 38.5 71) (width 0.2) (layer "B.Cu") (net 8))
 (segment (start 52.5 54.54) (end 60.25 46.79) (width 0.2) (layer "B.Cu") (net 8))
 (segment (start 54.29 118.92) (end 57.1885 118.92) (width 0.2) (layer "F.Cu") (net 15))
 (segment (start 57.1885 118.92) (end 63.5 125.2315) (width 0.2) (layer "F.Cu") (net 15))
 (segment (start 80.4985 71.92) (end 87 78.4215) (width 0.2) (layer "F.Cu") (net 18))
 (segment (start 77.79 71.92) (end 80.4985 71.92) (width 0.2) (layer "F.Cu") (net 18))
 (segment (start 80.6885 95.42) (end 87 101.7315) (width 0.2) (layer "F.Cu") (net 6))
 (segment (start 77.79 95.42) (end 80.6885 95.42) (width 0.2) (layer "F.Cu") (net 6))
 (segment (start 80.6885 118.92) (end 87 125.2315) (width 0.2) (layer "F.Cu") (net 14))
 (segment (start 77.79 118.92) (end 80.6885 118.92) (width 0.2) (layer "F.Cu") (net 14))
 (segment (start 104.9385 95.42) (end 111 101.4815) (width 0.2) (layer "F.Cu") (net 16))
 (segment (start 101.29 95.42) (end 104.9385 95.42) (width 0.2) (layer "F.Cu") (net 16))
 (segment (start 65 48) (end 65 55.5) (width 0.2) (layer "F.Cu") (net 20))
 (segment (start 65 55.5) (end 63.55 56.95) (width 0.2) (layer "F.Cu") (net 20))
 (segment (start 63.55 56.95) (end 60.25 56.95) (width 0.2) (layer "F.Cu") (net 20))
 (segment (start 107 55.71) (end 110.29 55.71) (width 0.2) (layer "F.Cu") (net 20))
 (segment (start 112.25 47.75) (end 109.75 45.25) (width 0.2) (layer "F.Cu") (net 20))
 (segment (start 112.25 53.75) (end 112.25 47.75) (width 0.2) (layer "F.Cu") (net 20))
 (segment (start 109.75 45.25) (end 67.75 45.25) (width 0.2) (layer "F.Cu") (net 20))
 (segment (start 67.75 45.25) (end 65 48) (width 0.2) (layer "F.Cu") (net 20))
 (segment (start 110.29 55.71) (end 112.25 53.75) (width 0.2) (layer "F.Cu") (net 20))
 (segment (start 55.75 52.25) (end 57.91 54.41) (width 0.2) (layer "F.Cu") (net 21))
 (segment (start 55.75 43.75) (end 55.75 52.25) (width 0.2) (layer "F.Cu") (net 21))
 (segment (start 110 58.25) (end 113.5 54.75) (width 0.2) (layer "F.Cu") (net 21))
 (segment (start 109.25 42.5) (end 57 42.5) (width 0.2) (layer "F.Cu") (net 21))
 (segment (start 57 42.5) (end 55.75 43.75) (width 0.2) (layer "F.Cu") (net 21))
 (segment (start 57.91 54.41) (end 60.25 54.41) (width 0.2) (layer "F.Cu") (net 21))
 (segment (start 113.5 54.75) (end 113.5 46.75) (width 0.2) (layer "F.Cu") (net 21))
 (segment (start 113.5 46.75) (end 109.25 42.5) (width 0.2) (layer "F.Cu") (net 21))
 (segment (start 107 58.25) (end 110 58.25) (width 0.2) (layer "F.Cu") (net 21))
 (segment (start 65 42.5) (end 46.765 42.5) (width 0.2) (layer "B.Cu") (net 19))
 (segment (start 46.765 42.5) (end 45.015 44.25) (width 0.2) (layer "B.Cu") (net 19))
 (segment (start 107 53.17) (end 75.67 53.17) (width 0.2) (layer "B.Cu") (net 19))
 (segment (start 75.67 53.17) (end 65 42.5) (width 0.2) (layer "B.Cu") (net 19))
 (segment (start 54.29 95.42) (end 57.1885 95.42) (width 0.2) (layer "F.Cu") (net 4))
 (segment (start 57.1885 95.42) (end 63.5 101.7315) (width 0.2) (layer "F.Cu") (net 4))
 (segment (start 45 74.75) (end 41.5 78.25) (width 0.2) (layer "F.Cu") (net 11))
 (segment (start 41.5 78.25) (end 41.5 79.0415) (width 0.2) (layer "F.Cu") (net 11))
 (segment (start 107.6015 78.2315) (end 110.75 78.2315) (width 0.2) (layer "F.Cu") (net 2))
 (segment (start 101.29 71.92) (end 107.6015 78.2315) (width 0.2) (layer "F.Cu") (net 2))
 (segment (start 101.29 118.92) (end 107.6015 125.2315) (width 0.2) (layer "F.Cu") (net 12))
 (segment (start 107.6015 125.2315) (end 110.75 125.2315) (width 0.2) (layer "F.Cu") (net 12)))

